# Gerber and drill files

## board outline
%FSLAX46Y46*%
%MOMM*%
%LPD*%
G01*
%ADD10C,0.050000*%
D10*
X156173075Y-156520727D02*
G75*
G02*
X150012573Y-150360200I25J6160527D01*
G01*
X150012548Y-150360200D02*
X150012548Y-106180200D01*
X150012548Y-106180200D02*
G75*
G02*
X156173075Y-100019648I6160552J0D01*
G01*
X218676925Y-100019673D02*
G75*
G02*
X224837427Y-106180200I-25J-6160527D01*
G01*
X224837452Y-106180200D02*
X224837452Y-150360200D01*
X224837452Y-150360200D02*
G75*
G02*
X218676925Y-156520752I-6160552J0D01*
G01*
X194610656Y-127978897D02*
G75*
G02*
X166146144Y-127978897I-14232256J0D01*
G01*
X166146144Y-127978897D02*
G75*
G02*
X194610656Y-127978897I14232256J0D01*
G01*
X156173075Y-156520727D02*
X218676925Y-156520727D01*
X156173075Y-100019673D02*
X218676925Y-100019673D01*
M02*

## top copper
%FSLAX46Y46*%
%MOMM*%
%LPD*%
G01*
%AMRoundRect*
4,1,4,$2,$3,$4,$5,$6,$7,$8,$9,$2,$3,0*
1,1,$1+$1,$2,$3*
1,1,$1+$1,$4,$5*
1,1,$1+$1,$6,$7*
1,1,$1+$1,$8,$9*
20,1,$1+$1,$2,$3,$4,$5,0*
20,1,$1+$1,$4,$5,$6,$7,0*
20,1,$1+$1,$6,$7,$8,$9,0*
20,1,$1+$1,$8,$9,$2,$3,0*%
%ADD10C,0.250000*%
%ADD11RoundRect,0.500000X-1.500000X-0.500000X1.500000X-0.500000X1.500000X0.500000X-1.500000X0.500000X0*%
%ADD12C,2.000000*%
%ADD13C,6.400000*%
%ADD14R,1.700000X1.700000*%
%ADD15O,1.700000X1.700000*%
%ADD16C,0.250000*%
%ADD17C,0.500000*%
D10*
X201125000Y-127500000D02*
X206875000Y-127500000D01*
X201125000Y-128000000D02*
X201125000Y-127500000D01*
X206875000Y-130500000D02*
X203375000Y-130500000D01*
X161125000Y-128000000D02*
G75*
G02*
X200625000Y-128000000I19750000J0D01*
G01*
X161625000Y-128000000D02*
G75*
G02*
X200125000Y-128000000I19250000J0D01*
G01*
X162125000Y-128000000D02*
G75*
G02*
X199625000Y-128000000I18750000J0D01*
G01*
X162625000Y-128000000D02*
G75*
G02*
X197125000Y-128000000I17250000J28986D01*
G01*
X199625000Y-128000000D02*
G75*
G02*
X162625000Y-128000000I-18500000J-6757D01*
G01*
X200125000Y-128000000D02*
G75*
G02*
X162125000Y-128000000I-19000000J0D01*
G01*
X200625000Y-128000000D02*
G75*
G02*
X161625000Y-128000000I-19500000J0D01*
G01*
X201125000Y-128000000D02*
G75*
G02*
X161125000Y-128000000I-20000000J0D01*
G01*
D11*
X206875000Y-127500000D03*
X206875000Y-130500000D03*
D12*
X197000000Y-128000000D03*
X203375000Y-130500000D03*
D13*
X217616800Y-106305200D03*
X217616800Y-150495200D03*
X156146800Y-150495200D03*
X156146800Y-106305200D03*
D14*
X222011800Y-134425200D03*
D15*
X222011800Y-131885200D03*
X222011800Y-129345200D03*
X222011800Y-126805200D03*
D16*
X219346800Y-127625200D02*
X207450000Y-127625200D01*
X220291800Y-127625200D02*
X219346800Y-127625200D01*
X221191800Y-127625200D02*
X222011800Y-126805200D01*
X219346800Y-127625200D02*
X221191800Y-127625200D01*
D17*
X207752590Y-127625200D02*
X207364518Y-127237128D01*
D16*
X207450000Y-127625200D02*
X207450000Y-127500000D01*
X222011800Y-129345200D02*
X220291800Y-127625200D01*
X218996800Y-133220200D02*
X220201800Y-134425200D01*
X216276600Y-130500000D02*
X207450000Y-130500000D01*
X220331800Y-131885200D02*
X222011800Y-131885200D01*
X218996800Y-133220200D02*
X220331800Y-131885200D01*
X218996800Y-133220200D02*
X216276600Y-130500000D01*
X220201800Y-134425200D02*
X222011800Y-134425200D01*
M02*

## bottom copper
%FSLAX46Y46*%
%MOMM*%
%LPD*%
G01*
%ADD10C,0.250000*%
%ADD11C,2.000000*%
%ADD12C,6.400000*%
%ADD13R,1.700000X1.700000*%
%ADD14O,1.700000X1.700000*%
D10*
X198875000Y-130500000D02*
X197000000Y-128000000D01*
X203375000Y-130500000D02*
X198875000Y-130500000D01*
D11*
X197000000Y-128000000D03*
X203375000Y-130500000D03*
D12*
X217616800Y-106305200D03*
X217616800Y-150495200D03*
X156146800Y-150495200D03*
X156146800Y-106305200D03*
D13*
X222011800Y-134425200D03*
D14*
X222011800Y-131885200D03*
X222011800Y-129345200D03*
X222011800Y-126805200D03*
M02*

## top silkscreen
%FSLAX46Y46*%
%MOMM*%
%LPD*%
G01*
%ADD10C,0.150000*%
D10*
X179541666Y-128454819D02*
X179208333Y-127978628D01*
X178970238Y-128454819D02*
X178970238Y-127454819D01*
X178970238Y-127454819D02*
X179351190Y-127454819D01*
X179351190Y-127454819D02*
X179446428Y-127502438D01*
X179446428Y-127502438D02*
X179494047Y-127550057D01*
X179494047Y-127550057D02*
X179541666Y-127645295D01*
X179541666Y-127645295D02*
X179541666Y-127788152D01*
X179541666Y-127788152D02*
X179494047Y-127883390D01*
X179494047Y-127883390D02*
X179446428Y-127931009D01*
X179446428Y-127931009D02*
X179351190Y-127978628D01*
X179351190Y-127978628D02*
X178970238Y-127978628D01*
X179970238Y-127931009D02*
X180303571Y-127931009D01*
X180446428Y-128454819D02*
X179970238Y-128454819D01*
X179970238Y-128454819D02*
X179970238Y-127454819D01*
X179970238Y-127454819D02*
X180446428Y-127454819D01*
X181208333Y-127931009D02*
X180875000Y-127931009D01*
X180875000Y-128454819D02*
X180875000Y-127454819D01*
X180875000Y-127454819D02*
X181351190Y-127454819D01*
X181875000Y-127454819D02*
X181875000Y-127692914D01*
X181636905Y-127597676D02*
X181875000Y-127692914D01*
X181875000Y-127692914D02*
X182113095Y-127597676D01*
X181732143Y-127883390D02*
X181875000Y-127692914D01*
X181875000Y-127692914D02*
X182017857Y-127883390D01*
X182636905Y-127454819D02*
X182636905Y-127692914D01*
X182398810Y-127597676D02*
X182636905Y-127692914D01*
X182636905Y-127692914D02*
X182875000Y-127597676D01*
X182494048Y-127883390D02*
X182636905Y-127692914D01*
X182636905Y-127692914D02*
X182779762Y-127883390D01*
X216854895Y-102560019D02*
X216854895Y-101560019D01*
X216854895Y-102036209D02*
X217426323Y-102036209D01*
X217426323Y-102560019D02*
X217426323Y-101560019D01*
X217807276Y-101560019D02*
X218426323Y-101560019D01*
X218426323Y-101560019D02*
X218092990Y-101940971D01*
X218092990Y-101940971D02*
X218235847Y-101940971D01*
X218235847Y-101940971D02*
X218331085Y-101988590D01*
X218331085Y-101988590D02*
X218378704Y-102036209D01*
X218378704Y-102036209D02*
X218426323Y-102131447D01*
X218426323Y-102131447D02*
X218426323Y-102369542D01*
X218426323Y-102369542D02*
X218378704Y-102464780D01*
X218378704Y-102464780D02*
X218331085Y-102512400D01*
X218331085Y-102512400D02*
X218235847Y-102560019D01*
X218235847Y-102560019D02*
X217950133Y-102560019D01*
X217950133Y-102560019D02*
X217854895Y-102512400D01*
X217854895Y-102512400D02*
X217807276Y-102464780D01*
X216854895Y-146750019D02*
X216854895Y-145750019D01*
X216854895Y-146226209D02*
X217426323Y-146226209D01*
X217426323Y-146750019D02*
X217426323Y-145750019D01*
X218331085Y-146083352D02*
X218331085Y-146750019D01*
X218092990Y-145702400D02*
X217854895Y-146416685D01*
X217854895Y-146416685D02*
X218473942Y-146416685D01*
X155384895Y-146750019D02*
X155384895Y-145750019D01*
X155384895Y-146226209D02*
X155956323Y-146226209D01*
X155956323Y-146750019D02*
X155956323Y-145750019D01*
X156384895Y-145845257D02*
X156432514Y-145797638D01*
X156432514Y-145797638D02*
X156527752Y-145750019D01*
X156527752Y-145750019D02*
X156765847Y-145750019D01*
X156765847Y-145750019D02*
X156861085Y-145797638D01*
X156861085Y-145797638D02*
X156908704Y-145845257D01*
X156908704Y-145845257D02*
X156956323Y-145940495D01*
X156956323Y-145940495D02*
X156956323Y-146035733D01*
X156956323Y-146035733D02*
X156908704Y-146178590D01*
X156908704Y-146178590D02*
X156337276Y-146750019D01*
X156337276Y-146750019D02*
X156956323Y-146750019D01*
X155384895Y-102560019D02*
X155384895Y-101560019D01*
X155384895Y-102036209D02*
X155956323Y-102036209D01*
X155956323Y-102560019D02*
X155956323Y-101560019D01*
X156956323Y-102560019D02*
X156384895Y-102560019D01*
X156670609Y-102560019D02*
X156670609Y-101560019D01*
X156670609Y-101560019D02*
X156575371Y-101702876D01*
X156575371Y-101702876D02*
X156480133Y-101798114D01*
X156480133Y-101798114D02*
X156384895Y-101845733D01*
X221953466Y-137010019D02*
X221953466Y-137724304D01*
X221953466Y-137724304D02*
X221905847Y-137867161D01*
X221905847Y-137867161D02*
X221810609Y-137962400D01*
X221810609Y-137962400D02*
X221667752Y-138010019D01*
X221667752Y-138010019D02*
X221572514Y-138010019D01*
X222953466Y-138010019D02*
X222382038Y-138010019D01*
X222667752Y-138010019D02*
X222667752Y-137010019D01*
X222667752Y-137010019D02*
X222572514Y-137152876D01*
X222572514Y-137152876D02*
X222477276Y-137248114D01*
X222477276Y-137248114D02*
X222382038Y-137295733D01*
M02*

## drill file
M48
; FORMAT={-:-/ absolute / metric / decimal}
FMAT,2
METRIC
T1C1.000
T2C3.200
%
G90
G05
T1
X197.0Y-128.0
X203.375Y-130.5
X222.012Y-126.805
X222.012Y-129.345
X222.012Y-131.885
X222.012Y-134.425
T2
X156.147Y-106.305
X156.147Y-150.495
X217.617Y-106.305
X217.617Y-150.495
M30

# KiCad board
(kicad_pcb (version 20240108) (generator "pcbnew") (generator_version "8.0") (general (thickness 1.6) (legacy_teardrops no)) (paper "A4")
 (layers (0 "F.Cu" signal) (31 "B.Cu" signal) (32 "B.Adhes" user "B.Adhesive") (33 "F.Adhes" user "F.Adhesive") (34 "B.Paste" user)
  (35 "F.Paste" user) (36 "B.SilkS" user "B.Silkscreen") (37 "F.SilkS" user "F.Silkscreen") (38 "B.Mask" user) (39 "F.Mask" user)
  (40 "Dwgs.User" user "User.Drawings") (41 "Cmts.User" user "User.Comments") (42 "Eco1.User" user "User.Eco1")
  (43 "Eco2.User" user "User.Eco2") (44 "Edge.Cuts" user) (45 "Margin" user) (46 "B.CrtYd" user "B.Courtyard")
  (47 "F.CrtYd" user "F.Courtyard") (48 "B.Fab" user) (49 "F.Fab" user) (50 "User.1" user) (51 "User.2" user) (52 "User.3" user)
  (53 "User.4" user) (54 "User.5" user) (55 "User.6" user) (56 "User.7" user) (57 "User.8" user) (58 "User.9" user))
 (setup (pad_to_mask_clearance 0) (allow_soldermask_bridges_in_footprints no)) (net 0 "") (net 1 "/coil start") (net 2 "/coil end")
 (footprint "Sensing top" (layer "F.Cu") (at 180.875 128)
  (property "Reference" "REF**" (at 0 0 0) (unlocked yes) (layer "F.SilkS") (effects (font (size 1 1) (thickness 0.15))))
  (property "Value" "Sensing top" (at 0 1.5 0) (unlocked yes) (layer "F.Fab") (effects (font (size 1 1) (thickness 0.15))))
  (fp_line (start 20.25 -0.5) (end 26 -0.5) (stroke (width 0.25) (type solid)) (layer "F.Cu"))
  (fp_line (start 20.25 0) (end 20.25 -0.5) (stroke (width 0.25) (type solid)) (layer "F.Cu"))
  (fp_line (start 26 2.5) (end 22.5 2.5) (stroke (width 0.25) (type default)) (layer "F.Cu"))
  (fp_arc (start -19.75 0) (mid 0 -19.75) (end 19.75 0) (stroke (width 0.25) (type solid)) (layer "F.Cu"))
  (fp_arc (start -19.25 0) (mid 0 -19.25) (end 19.25 0) (stroke (width 0.25) (type solid)) (layer "F.Cu"))
  (fp_arc (start -18.75 0) (mid 0 -18.75) (end 18.75 0) (stroke (width 0.25) (type solid)) (layer "F.Cu"))
  (fp_arc (start -18.25 0) (mid -1 -17.27901) (end 16.25 0) (stroke (width 0.25) (type solid)) (layer "F.Cu"))
  (fp_arc (start 18.75 0) (mid 0.25 18.506758) (end -18.25 0) (stroke (width 0.25) (type solid)) (layer "F.Cu"))
  (fp_arc (start 19.25 0) (mid 0.25 19) (end -18.75 0) (stroke (width 0.25) (type solid)) (layer "F.Cu"))
  (fp_arc (start 19.75 0) (mid 0.25 19.5) (end -19.25 0) (stroke (width 0.25) (type solid)) (layer "F.Cu"))
  (fp_arc (start 20.25 0) (mid 0.25 20) (end -19.75 0) (stroke (width 0.25) (type solid)) (layer "F.Cu"))
  (fp_line (start 18 2.5) (end 16.125 0) (stroke (width 0.25) (type default)) (layer "B.Cu"))
  (fp_line (start 22.5 2.5) (end 18 2.5) (stroke (width 0.25) (type default)) (layer "B.Cu"))
  (pad "1" smd roundrect (at 26 -0.5) (size 4 2) (layers "F.Cu") (roundrect_rratio 0.25) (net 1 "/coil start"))
  (pad "2" smd roundrect (at 26 2.5) (size 4 2) (layers "F.Cu") (roundrect_rratio 0.25) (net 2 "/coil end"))
  (pad "3" thru_hole circle (at 16.125 0) (size 2 2) (drill 1) (layers "*.Cu" "*.Mask") (remove_unused_layers no))
  (pad "3" thru_hole circle (at 22.5 2.5) (size 2 2) (drill 1) (layers "*.Cu" "*.Mask") (remove_unused_layers no)))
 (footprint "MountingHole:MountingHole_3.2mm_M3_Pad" (layer "F.Cu") (at 217.6168 106.3052)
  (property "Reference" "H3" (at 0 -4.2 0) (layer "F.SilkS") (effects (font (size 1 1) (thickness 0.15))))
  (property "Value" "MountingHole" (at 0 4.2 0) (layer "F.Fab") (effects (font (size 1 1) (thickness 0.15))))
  (pad "1" thru_hole circle (at 0 0) (size 6.4 6.4) (drill 3.2) (layers "*.Cu" "*.Mask") (remove_unused_layers no)))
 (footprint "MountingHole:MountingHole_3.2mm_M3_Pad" (layer "F.Cu") (at 217.6168 150.4952)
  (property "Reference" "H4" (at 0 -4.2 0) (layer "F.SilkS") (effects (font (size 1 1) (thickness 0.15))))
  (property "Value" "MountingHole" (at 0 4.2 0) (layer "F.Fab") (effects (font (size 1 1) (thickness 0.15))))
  (pad "1" thru_hole circle (at 0 0) (size 6.4 6.4) (drill 3.2) (layers "*.Cu" "*.Mask") (remove_unused_layers no)))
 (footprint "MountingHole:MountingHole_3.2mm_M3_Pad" (layer "F.Cu") (at 156.1468 150.4952)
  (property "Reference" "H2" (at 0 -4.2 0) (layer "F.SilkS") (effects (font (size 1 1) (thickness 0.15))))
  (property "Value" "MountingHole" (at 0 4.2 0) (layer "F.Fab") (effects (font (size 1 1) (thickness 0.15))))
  (pad "1" thru_hole circle (at 0 0) (size 6.4 6.4) (drill 3.2) (layers "*.Cu" "*.Mask") (remove_unused_layers no)))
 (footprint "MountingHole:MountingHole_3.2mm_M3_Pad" (layer "F.Cu") (at 156.1468 106.3052)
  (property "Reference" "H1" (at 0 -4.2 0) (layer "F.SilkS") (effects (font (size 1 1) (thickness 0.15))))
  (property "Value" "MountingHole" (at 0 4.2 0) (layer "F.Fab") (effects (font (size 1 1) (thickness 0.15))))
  (pad "1" thru_hole circle (at 0 0) (size 6.4 6.4) (drill 3.2) (layers "*.Cu" "*.Mask") (remove_unused_layers no)))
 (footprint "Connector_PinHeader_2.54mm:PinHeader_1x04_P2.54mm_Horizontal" (layer "B.Cu") (at 222.0118 134.4252)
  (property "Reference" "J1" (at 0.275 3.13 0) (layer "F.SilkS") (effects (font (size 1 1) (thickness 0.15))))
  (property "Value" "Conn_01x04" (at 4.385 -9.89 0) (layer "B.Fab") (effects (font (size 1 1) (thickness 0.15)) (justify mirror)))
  (pad "1" thru_hole rect (at 0 0) (size 1.7 1.7) (drill 1) (layers "*.Cu" "*.Mask") (remove_unused_layers no) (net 2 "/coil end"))
  (pad "2" thru_hole oval (at 0 -2.54) (size 1.7 1.7) (drill 1) (layers "*.Cu" "*.Mask") (remove_unused_layers no) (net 2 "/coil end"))
  (pad "3" thru_hole oval (at 0 -5.08) (size 1.7 1.7) (drill 1) (layers "*.Cu" "*.Mask") (remove_unused_layers no) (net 1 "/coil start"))
  (pad "4" thru_hole oval (at 0 -7.62) (size 1.7 1.7) (drill 1) (layers "*.Cu" "*.Mask") (remove_unused_layers no) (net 1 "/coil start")))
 (gr_arc (start 156.173075 156.520727) (mid 151.816925 154.71635) (end 150.012548 150.3602) (stroke (width 0.05) (type default))
  (layer "Edge.Cuts"))
 (gr_line (start 150.012548 150.3602) (end 150.012548 106.1802) (stroke (width 0.05) (type default)) (layer "Edge.Cuts"))
 (gr_arc (start 150.012548 106.1802) (mid 151.816925 101.82405) (end 156.173075 100.019673) (stroke (width 0.05) (type default))
  (layer "Edge.Cuts"))
 (gr_arc (start 218.676925 100.019673) (mid 223.033075 101.82405) (end 224.837452 106.1802) (stroke (width 0.05) (type default))
  (layer "Edge.Cuts"))
 (gr_line (start 224.837452 106.1802) (end 224.837452 150.3602) (stroke (width 0.05) (type default)) (layer "Edge.Cuts"))
 (gr_arc (start 224.837452 150.3602) (mid 223.033075 154.71635) (end 218.676925 156.520727) (stroke (width 0.05) (type default))
  (layer "Edge.Cuts"))
 (gr_circle (center 180.3784 127.978897) (end 192.7568 120.9552) (stroke (width 0.05) (type default)) (fill none) (layer "Edge.Cuts"))
 (gr_line (start 156.173075 156.520727) (end 218.676925 156.520727) (stroke (width 0.05) (type default)) (layer "Edge.Cuts"))
 (gr_line (start 156.173075 100.019673) (end 218.676925 100.019673) (stroke (width 0.05) (type default)) (layer "Edge.Cuts"))
 (segment (start 219.3468 127.6252) (end 207.45 127.6252) (width 0.25) (layer "F.Cu") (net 1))
 (segment (start 220.2918 127.6252) (end 219.3468 127.6252) (width 0.25) (layer "F.Cu") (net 1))
 (segment (start 221.1918 127.6252) (end 222.0118 126.8052) (width 0.25) (layer "F.Cu") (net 1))
 (segment (start 219.3468 127.6252) (end 221.1918 127.6252) (width 0.25) (layer "F.Cu") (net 1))
 (segment (start 207.75259 127.6252) (end 207.364518 127.237128) (width 0.5) (layer "F.Cu") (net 1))
 (segment (start 207.45 127.6252) (end 207.45 127.5) (width 0.25) (layer "F.Cu") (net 1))
 (segment (start 222.0118 129.3452) (end 220.2918 127.6252) (width 0.25) (layer "F.Cu") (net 1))
 (segment (start 218.9968 133.2202) (end 220.2018 134.4252) (width 0.25) (layer "F.Cu") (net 2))
 (segment (start 216.2766 130.5) (end 207.45 130.5) (width 0.25) (layer "F.Cu") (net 2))
 (segment (start 220.3318 131.8852) (end 222.0118 131.8852) (width 0.25) (layer "F.Cu") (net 2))
 (segment (start 218.9968 133.2202) (end 220.3318 131.8852) (width 0.25) (layer "F.Cu") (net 2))
 (segment (start 218.9968 133.2202) (end 216.2766 130.5) (width 0.25) (layer "F.Cu") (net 2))
 (segment (start 220.2018 134.4252) (end 222.0118 134.4252) (width 0.25) (layer "F.Cu") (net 2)))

